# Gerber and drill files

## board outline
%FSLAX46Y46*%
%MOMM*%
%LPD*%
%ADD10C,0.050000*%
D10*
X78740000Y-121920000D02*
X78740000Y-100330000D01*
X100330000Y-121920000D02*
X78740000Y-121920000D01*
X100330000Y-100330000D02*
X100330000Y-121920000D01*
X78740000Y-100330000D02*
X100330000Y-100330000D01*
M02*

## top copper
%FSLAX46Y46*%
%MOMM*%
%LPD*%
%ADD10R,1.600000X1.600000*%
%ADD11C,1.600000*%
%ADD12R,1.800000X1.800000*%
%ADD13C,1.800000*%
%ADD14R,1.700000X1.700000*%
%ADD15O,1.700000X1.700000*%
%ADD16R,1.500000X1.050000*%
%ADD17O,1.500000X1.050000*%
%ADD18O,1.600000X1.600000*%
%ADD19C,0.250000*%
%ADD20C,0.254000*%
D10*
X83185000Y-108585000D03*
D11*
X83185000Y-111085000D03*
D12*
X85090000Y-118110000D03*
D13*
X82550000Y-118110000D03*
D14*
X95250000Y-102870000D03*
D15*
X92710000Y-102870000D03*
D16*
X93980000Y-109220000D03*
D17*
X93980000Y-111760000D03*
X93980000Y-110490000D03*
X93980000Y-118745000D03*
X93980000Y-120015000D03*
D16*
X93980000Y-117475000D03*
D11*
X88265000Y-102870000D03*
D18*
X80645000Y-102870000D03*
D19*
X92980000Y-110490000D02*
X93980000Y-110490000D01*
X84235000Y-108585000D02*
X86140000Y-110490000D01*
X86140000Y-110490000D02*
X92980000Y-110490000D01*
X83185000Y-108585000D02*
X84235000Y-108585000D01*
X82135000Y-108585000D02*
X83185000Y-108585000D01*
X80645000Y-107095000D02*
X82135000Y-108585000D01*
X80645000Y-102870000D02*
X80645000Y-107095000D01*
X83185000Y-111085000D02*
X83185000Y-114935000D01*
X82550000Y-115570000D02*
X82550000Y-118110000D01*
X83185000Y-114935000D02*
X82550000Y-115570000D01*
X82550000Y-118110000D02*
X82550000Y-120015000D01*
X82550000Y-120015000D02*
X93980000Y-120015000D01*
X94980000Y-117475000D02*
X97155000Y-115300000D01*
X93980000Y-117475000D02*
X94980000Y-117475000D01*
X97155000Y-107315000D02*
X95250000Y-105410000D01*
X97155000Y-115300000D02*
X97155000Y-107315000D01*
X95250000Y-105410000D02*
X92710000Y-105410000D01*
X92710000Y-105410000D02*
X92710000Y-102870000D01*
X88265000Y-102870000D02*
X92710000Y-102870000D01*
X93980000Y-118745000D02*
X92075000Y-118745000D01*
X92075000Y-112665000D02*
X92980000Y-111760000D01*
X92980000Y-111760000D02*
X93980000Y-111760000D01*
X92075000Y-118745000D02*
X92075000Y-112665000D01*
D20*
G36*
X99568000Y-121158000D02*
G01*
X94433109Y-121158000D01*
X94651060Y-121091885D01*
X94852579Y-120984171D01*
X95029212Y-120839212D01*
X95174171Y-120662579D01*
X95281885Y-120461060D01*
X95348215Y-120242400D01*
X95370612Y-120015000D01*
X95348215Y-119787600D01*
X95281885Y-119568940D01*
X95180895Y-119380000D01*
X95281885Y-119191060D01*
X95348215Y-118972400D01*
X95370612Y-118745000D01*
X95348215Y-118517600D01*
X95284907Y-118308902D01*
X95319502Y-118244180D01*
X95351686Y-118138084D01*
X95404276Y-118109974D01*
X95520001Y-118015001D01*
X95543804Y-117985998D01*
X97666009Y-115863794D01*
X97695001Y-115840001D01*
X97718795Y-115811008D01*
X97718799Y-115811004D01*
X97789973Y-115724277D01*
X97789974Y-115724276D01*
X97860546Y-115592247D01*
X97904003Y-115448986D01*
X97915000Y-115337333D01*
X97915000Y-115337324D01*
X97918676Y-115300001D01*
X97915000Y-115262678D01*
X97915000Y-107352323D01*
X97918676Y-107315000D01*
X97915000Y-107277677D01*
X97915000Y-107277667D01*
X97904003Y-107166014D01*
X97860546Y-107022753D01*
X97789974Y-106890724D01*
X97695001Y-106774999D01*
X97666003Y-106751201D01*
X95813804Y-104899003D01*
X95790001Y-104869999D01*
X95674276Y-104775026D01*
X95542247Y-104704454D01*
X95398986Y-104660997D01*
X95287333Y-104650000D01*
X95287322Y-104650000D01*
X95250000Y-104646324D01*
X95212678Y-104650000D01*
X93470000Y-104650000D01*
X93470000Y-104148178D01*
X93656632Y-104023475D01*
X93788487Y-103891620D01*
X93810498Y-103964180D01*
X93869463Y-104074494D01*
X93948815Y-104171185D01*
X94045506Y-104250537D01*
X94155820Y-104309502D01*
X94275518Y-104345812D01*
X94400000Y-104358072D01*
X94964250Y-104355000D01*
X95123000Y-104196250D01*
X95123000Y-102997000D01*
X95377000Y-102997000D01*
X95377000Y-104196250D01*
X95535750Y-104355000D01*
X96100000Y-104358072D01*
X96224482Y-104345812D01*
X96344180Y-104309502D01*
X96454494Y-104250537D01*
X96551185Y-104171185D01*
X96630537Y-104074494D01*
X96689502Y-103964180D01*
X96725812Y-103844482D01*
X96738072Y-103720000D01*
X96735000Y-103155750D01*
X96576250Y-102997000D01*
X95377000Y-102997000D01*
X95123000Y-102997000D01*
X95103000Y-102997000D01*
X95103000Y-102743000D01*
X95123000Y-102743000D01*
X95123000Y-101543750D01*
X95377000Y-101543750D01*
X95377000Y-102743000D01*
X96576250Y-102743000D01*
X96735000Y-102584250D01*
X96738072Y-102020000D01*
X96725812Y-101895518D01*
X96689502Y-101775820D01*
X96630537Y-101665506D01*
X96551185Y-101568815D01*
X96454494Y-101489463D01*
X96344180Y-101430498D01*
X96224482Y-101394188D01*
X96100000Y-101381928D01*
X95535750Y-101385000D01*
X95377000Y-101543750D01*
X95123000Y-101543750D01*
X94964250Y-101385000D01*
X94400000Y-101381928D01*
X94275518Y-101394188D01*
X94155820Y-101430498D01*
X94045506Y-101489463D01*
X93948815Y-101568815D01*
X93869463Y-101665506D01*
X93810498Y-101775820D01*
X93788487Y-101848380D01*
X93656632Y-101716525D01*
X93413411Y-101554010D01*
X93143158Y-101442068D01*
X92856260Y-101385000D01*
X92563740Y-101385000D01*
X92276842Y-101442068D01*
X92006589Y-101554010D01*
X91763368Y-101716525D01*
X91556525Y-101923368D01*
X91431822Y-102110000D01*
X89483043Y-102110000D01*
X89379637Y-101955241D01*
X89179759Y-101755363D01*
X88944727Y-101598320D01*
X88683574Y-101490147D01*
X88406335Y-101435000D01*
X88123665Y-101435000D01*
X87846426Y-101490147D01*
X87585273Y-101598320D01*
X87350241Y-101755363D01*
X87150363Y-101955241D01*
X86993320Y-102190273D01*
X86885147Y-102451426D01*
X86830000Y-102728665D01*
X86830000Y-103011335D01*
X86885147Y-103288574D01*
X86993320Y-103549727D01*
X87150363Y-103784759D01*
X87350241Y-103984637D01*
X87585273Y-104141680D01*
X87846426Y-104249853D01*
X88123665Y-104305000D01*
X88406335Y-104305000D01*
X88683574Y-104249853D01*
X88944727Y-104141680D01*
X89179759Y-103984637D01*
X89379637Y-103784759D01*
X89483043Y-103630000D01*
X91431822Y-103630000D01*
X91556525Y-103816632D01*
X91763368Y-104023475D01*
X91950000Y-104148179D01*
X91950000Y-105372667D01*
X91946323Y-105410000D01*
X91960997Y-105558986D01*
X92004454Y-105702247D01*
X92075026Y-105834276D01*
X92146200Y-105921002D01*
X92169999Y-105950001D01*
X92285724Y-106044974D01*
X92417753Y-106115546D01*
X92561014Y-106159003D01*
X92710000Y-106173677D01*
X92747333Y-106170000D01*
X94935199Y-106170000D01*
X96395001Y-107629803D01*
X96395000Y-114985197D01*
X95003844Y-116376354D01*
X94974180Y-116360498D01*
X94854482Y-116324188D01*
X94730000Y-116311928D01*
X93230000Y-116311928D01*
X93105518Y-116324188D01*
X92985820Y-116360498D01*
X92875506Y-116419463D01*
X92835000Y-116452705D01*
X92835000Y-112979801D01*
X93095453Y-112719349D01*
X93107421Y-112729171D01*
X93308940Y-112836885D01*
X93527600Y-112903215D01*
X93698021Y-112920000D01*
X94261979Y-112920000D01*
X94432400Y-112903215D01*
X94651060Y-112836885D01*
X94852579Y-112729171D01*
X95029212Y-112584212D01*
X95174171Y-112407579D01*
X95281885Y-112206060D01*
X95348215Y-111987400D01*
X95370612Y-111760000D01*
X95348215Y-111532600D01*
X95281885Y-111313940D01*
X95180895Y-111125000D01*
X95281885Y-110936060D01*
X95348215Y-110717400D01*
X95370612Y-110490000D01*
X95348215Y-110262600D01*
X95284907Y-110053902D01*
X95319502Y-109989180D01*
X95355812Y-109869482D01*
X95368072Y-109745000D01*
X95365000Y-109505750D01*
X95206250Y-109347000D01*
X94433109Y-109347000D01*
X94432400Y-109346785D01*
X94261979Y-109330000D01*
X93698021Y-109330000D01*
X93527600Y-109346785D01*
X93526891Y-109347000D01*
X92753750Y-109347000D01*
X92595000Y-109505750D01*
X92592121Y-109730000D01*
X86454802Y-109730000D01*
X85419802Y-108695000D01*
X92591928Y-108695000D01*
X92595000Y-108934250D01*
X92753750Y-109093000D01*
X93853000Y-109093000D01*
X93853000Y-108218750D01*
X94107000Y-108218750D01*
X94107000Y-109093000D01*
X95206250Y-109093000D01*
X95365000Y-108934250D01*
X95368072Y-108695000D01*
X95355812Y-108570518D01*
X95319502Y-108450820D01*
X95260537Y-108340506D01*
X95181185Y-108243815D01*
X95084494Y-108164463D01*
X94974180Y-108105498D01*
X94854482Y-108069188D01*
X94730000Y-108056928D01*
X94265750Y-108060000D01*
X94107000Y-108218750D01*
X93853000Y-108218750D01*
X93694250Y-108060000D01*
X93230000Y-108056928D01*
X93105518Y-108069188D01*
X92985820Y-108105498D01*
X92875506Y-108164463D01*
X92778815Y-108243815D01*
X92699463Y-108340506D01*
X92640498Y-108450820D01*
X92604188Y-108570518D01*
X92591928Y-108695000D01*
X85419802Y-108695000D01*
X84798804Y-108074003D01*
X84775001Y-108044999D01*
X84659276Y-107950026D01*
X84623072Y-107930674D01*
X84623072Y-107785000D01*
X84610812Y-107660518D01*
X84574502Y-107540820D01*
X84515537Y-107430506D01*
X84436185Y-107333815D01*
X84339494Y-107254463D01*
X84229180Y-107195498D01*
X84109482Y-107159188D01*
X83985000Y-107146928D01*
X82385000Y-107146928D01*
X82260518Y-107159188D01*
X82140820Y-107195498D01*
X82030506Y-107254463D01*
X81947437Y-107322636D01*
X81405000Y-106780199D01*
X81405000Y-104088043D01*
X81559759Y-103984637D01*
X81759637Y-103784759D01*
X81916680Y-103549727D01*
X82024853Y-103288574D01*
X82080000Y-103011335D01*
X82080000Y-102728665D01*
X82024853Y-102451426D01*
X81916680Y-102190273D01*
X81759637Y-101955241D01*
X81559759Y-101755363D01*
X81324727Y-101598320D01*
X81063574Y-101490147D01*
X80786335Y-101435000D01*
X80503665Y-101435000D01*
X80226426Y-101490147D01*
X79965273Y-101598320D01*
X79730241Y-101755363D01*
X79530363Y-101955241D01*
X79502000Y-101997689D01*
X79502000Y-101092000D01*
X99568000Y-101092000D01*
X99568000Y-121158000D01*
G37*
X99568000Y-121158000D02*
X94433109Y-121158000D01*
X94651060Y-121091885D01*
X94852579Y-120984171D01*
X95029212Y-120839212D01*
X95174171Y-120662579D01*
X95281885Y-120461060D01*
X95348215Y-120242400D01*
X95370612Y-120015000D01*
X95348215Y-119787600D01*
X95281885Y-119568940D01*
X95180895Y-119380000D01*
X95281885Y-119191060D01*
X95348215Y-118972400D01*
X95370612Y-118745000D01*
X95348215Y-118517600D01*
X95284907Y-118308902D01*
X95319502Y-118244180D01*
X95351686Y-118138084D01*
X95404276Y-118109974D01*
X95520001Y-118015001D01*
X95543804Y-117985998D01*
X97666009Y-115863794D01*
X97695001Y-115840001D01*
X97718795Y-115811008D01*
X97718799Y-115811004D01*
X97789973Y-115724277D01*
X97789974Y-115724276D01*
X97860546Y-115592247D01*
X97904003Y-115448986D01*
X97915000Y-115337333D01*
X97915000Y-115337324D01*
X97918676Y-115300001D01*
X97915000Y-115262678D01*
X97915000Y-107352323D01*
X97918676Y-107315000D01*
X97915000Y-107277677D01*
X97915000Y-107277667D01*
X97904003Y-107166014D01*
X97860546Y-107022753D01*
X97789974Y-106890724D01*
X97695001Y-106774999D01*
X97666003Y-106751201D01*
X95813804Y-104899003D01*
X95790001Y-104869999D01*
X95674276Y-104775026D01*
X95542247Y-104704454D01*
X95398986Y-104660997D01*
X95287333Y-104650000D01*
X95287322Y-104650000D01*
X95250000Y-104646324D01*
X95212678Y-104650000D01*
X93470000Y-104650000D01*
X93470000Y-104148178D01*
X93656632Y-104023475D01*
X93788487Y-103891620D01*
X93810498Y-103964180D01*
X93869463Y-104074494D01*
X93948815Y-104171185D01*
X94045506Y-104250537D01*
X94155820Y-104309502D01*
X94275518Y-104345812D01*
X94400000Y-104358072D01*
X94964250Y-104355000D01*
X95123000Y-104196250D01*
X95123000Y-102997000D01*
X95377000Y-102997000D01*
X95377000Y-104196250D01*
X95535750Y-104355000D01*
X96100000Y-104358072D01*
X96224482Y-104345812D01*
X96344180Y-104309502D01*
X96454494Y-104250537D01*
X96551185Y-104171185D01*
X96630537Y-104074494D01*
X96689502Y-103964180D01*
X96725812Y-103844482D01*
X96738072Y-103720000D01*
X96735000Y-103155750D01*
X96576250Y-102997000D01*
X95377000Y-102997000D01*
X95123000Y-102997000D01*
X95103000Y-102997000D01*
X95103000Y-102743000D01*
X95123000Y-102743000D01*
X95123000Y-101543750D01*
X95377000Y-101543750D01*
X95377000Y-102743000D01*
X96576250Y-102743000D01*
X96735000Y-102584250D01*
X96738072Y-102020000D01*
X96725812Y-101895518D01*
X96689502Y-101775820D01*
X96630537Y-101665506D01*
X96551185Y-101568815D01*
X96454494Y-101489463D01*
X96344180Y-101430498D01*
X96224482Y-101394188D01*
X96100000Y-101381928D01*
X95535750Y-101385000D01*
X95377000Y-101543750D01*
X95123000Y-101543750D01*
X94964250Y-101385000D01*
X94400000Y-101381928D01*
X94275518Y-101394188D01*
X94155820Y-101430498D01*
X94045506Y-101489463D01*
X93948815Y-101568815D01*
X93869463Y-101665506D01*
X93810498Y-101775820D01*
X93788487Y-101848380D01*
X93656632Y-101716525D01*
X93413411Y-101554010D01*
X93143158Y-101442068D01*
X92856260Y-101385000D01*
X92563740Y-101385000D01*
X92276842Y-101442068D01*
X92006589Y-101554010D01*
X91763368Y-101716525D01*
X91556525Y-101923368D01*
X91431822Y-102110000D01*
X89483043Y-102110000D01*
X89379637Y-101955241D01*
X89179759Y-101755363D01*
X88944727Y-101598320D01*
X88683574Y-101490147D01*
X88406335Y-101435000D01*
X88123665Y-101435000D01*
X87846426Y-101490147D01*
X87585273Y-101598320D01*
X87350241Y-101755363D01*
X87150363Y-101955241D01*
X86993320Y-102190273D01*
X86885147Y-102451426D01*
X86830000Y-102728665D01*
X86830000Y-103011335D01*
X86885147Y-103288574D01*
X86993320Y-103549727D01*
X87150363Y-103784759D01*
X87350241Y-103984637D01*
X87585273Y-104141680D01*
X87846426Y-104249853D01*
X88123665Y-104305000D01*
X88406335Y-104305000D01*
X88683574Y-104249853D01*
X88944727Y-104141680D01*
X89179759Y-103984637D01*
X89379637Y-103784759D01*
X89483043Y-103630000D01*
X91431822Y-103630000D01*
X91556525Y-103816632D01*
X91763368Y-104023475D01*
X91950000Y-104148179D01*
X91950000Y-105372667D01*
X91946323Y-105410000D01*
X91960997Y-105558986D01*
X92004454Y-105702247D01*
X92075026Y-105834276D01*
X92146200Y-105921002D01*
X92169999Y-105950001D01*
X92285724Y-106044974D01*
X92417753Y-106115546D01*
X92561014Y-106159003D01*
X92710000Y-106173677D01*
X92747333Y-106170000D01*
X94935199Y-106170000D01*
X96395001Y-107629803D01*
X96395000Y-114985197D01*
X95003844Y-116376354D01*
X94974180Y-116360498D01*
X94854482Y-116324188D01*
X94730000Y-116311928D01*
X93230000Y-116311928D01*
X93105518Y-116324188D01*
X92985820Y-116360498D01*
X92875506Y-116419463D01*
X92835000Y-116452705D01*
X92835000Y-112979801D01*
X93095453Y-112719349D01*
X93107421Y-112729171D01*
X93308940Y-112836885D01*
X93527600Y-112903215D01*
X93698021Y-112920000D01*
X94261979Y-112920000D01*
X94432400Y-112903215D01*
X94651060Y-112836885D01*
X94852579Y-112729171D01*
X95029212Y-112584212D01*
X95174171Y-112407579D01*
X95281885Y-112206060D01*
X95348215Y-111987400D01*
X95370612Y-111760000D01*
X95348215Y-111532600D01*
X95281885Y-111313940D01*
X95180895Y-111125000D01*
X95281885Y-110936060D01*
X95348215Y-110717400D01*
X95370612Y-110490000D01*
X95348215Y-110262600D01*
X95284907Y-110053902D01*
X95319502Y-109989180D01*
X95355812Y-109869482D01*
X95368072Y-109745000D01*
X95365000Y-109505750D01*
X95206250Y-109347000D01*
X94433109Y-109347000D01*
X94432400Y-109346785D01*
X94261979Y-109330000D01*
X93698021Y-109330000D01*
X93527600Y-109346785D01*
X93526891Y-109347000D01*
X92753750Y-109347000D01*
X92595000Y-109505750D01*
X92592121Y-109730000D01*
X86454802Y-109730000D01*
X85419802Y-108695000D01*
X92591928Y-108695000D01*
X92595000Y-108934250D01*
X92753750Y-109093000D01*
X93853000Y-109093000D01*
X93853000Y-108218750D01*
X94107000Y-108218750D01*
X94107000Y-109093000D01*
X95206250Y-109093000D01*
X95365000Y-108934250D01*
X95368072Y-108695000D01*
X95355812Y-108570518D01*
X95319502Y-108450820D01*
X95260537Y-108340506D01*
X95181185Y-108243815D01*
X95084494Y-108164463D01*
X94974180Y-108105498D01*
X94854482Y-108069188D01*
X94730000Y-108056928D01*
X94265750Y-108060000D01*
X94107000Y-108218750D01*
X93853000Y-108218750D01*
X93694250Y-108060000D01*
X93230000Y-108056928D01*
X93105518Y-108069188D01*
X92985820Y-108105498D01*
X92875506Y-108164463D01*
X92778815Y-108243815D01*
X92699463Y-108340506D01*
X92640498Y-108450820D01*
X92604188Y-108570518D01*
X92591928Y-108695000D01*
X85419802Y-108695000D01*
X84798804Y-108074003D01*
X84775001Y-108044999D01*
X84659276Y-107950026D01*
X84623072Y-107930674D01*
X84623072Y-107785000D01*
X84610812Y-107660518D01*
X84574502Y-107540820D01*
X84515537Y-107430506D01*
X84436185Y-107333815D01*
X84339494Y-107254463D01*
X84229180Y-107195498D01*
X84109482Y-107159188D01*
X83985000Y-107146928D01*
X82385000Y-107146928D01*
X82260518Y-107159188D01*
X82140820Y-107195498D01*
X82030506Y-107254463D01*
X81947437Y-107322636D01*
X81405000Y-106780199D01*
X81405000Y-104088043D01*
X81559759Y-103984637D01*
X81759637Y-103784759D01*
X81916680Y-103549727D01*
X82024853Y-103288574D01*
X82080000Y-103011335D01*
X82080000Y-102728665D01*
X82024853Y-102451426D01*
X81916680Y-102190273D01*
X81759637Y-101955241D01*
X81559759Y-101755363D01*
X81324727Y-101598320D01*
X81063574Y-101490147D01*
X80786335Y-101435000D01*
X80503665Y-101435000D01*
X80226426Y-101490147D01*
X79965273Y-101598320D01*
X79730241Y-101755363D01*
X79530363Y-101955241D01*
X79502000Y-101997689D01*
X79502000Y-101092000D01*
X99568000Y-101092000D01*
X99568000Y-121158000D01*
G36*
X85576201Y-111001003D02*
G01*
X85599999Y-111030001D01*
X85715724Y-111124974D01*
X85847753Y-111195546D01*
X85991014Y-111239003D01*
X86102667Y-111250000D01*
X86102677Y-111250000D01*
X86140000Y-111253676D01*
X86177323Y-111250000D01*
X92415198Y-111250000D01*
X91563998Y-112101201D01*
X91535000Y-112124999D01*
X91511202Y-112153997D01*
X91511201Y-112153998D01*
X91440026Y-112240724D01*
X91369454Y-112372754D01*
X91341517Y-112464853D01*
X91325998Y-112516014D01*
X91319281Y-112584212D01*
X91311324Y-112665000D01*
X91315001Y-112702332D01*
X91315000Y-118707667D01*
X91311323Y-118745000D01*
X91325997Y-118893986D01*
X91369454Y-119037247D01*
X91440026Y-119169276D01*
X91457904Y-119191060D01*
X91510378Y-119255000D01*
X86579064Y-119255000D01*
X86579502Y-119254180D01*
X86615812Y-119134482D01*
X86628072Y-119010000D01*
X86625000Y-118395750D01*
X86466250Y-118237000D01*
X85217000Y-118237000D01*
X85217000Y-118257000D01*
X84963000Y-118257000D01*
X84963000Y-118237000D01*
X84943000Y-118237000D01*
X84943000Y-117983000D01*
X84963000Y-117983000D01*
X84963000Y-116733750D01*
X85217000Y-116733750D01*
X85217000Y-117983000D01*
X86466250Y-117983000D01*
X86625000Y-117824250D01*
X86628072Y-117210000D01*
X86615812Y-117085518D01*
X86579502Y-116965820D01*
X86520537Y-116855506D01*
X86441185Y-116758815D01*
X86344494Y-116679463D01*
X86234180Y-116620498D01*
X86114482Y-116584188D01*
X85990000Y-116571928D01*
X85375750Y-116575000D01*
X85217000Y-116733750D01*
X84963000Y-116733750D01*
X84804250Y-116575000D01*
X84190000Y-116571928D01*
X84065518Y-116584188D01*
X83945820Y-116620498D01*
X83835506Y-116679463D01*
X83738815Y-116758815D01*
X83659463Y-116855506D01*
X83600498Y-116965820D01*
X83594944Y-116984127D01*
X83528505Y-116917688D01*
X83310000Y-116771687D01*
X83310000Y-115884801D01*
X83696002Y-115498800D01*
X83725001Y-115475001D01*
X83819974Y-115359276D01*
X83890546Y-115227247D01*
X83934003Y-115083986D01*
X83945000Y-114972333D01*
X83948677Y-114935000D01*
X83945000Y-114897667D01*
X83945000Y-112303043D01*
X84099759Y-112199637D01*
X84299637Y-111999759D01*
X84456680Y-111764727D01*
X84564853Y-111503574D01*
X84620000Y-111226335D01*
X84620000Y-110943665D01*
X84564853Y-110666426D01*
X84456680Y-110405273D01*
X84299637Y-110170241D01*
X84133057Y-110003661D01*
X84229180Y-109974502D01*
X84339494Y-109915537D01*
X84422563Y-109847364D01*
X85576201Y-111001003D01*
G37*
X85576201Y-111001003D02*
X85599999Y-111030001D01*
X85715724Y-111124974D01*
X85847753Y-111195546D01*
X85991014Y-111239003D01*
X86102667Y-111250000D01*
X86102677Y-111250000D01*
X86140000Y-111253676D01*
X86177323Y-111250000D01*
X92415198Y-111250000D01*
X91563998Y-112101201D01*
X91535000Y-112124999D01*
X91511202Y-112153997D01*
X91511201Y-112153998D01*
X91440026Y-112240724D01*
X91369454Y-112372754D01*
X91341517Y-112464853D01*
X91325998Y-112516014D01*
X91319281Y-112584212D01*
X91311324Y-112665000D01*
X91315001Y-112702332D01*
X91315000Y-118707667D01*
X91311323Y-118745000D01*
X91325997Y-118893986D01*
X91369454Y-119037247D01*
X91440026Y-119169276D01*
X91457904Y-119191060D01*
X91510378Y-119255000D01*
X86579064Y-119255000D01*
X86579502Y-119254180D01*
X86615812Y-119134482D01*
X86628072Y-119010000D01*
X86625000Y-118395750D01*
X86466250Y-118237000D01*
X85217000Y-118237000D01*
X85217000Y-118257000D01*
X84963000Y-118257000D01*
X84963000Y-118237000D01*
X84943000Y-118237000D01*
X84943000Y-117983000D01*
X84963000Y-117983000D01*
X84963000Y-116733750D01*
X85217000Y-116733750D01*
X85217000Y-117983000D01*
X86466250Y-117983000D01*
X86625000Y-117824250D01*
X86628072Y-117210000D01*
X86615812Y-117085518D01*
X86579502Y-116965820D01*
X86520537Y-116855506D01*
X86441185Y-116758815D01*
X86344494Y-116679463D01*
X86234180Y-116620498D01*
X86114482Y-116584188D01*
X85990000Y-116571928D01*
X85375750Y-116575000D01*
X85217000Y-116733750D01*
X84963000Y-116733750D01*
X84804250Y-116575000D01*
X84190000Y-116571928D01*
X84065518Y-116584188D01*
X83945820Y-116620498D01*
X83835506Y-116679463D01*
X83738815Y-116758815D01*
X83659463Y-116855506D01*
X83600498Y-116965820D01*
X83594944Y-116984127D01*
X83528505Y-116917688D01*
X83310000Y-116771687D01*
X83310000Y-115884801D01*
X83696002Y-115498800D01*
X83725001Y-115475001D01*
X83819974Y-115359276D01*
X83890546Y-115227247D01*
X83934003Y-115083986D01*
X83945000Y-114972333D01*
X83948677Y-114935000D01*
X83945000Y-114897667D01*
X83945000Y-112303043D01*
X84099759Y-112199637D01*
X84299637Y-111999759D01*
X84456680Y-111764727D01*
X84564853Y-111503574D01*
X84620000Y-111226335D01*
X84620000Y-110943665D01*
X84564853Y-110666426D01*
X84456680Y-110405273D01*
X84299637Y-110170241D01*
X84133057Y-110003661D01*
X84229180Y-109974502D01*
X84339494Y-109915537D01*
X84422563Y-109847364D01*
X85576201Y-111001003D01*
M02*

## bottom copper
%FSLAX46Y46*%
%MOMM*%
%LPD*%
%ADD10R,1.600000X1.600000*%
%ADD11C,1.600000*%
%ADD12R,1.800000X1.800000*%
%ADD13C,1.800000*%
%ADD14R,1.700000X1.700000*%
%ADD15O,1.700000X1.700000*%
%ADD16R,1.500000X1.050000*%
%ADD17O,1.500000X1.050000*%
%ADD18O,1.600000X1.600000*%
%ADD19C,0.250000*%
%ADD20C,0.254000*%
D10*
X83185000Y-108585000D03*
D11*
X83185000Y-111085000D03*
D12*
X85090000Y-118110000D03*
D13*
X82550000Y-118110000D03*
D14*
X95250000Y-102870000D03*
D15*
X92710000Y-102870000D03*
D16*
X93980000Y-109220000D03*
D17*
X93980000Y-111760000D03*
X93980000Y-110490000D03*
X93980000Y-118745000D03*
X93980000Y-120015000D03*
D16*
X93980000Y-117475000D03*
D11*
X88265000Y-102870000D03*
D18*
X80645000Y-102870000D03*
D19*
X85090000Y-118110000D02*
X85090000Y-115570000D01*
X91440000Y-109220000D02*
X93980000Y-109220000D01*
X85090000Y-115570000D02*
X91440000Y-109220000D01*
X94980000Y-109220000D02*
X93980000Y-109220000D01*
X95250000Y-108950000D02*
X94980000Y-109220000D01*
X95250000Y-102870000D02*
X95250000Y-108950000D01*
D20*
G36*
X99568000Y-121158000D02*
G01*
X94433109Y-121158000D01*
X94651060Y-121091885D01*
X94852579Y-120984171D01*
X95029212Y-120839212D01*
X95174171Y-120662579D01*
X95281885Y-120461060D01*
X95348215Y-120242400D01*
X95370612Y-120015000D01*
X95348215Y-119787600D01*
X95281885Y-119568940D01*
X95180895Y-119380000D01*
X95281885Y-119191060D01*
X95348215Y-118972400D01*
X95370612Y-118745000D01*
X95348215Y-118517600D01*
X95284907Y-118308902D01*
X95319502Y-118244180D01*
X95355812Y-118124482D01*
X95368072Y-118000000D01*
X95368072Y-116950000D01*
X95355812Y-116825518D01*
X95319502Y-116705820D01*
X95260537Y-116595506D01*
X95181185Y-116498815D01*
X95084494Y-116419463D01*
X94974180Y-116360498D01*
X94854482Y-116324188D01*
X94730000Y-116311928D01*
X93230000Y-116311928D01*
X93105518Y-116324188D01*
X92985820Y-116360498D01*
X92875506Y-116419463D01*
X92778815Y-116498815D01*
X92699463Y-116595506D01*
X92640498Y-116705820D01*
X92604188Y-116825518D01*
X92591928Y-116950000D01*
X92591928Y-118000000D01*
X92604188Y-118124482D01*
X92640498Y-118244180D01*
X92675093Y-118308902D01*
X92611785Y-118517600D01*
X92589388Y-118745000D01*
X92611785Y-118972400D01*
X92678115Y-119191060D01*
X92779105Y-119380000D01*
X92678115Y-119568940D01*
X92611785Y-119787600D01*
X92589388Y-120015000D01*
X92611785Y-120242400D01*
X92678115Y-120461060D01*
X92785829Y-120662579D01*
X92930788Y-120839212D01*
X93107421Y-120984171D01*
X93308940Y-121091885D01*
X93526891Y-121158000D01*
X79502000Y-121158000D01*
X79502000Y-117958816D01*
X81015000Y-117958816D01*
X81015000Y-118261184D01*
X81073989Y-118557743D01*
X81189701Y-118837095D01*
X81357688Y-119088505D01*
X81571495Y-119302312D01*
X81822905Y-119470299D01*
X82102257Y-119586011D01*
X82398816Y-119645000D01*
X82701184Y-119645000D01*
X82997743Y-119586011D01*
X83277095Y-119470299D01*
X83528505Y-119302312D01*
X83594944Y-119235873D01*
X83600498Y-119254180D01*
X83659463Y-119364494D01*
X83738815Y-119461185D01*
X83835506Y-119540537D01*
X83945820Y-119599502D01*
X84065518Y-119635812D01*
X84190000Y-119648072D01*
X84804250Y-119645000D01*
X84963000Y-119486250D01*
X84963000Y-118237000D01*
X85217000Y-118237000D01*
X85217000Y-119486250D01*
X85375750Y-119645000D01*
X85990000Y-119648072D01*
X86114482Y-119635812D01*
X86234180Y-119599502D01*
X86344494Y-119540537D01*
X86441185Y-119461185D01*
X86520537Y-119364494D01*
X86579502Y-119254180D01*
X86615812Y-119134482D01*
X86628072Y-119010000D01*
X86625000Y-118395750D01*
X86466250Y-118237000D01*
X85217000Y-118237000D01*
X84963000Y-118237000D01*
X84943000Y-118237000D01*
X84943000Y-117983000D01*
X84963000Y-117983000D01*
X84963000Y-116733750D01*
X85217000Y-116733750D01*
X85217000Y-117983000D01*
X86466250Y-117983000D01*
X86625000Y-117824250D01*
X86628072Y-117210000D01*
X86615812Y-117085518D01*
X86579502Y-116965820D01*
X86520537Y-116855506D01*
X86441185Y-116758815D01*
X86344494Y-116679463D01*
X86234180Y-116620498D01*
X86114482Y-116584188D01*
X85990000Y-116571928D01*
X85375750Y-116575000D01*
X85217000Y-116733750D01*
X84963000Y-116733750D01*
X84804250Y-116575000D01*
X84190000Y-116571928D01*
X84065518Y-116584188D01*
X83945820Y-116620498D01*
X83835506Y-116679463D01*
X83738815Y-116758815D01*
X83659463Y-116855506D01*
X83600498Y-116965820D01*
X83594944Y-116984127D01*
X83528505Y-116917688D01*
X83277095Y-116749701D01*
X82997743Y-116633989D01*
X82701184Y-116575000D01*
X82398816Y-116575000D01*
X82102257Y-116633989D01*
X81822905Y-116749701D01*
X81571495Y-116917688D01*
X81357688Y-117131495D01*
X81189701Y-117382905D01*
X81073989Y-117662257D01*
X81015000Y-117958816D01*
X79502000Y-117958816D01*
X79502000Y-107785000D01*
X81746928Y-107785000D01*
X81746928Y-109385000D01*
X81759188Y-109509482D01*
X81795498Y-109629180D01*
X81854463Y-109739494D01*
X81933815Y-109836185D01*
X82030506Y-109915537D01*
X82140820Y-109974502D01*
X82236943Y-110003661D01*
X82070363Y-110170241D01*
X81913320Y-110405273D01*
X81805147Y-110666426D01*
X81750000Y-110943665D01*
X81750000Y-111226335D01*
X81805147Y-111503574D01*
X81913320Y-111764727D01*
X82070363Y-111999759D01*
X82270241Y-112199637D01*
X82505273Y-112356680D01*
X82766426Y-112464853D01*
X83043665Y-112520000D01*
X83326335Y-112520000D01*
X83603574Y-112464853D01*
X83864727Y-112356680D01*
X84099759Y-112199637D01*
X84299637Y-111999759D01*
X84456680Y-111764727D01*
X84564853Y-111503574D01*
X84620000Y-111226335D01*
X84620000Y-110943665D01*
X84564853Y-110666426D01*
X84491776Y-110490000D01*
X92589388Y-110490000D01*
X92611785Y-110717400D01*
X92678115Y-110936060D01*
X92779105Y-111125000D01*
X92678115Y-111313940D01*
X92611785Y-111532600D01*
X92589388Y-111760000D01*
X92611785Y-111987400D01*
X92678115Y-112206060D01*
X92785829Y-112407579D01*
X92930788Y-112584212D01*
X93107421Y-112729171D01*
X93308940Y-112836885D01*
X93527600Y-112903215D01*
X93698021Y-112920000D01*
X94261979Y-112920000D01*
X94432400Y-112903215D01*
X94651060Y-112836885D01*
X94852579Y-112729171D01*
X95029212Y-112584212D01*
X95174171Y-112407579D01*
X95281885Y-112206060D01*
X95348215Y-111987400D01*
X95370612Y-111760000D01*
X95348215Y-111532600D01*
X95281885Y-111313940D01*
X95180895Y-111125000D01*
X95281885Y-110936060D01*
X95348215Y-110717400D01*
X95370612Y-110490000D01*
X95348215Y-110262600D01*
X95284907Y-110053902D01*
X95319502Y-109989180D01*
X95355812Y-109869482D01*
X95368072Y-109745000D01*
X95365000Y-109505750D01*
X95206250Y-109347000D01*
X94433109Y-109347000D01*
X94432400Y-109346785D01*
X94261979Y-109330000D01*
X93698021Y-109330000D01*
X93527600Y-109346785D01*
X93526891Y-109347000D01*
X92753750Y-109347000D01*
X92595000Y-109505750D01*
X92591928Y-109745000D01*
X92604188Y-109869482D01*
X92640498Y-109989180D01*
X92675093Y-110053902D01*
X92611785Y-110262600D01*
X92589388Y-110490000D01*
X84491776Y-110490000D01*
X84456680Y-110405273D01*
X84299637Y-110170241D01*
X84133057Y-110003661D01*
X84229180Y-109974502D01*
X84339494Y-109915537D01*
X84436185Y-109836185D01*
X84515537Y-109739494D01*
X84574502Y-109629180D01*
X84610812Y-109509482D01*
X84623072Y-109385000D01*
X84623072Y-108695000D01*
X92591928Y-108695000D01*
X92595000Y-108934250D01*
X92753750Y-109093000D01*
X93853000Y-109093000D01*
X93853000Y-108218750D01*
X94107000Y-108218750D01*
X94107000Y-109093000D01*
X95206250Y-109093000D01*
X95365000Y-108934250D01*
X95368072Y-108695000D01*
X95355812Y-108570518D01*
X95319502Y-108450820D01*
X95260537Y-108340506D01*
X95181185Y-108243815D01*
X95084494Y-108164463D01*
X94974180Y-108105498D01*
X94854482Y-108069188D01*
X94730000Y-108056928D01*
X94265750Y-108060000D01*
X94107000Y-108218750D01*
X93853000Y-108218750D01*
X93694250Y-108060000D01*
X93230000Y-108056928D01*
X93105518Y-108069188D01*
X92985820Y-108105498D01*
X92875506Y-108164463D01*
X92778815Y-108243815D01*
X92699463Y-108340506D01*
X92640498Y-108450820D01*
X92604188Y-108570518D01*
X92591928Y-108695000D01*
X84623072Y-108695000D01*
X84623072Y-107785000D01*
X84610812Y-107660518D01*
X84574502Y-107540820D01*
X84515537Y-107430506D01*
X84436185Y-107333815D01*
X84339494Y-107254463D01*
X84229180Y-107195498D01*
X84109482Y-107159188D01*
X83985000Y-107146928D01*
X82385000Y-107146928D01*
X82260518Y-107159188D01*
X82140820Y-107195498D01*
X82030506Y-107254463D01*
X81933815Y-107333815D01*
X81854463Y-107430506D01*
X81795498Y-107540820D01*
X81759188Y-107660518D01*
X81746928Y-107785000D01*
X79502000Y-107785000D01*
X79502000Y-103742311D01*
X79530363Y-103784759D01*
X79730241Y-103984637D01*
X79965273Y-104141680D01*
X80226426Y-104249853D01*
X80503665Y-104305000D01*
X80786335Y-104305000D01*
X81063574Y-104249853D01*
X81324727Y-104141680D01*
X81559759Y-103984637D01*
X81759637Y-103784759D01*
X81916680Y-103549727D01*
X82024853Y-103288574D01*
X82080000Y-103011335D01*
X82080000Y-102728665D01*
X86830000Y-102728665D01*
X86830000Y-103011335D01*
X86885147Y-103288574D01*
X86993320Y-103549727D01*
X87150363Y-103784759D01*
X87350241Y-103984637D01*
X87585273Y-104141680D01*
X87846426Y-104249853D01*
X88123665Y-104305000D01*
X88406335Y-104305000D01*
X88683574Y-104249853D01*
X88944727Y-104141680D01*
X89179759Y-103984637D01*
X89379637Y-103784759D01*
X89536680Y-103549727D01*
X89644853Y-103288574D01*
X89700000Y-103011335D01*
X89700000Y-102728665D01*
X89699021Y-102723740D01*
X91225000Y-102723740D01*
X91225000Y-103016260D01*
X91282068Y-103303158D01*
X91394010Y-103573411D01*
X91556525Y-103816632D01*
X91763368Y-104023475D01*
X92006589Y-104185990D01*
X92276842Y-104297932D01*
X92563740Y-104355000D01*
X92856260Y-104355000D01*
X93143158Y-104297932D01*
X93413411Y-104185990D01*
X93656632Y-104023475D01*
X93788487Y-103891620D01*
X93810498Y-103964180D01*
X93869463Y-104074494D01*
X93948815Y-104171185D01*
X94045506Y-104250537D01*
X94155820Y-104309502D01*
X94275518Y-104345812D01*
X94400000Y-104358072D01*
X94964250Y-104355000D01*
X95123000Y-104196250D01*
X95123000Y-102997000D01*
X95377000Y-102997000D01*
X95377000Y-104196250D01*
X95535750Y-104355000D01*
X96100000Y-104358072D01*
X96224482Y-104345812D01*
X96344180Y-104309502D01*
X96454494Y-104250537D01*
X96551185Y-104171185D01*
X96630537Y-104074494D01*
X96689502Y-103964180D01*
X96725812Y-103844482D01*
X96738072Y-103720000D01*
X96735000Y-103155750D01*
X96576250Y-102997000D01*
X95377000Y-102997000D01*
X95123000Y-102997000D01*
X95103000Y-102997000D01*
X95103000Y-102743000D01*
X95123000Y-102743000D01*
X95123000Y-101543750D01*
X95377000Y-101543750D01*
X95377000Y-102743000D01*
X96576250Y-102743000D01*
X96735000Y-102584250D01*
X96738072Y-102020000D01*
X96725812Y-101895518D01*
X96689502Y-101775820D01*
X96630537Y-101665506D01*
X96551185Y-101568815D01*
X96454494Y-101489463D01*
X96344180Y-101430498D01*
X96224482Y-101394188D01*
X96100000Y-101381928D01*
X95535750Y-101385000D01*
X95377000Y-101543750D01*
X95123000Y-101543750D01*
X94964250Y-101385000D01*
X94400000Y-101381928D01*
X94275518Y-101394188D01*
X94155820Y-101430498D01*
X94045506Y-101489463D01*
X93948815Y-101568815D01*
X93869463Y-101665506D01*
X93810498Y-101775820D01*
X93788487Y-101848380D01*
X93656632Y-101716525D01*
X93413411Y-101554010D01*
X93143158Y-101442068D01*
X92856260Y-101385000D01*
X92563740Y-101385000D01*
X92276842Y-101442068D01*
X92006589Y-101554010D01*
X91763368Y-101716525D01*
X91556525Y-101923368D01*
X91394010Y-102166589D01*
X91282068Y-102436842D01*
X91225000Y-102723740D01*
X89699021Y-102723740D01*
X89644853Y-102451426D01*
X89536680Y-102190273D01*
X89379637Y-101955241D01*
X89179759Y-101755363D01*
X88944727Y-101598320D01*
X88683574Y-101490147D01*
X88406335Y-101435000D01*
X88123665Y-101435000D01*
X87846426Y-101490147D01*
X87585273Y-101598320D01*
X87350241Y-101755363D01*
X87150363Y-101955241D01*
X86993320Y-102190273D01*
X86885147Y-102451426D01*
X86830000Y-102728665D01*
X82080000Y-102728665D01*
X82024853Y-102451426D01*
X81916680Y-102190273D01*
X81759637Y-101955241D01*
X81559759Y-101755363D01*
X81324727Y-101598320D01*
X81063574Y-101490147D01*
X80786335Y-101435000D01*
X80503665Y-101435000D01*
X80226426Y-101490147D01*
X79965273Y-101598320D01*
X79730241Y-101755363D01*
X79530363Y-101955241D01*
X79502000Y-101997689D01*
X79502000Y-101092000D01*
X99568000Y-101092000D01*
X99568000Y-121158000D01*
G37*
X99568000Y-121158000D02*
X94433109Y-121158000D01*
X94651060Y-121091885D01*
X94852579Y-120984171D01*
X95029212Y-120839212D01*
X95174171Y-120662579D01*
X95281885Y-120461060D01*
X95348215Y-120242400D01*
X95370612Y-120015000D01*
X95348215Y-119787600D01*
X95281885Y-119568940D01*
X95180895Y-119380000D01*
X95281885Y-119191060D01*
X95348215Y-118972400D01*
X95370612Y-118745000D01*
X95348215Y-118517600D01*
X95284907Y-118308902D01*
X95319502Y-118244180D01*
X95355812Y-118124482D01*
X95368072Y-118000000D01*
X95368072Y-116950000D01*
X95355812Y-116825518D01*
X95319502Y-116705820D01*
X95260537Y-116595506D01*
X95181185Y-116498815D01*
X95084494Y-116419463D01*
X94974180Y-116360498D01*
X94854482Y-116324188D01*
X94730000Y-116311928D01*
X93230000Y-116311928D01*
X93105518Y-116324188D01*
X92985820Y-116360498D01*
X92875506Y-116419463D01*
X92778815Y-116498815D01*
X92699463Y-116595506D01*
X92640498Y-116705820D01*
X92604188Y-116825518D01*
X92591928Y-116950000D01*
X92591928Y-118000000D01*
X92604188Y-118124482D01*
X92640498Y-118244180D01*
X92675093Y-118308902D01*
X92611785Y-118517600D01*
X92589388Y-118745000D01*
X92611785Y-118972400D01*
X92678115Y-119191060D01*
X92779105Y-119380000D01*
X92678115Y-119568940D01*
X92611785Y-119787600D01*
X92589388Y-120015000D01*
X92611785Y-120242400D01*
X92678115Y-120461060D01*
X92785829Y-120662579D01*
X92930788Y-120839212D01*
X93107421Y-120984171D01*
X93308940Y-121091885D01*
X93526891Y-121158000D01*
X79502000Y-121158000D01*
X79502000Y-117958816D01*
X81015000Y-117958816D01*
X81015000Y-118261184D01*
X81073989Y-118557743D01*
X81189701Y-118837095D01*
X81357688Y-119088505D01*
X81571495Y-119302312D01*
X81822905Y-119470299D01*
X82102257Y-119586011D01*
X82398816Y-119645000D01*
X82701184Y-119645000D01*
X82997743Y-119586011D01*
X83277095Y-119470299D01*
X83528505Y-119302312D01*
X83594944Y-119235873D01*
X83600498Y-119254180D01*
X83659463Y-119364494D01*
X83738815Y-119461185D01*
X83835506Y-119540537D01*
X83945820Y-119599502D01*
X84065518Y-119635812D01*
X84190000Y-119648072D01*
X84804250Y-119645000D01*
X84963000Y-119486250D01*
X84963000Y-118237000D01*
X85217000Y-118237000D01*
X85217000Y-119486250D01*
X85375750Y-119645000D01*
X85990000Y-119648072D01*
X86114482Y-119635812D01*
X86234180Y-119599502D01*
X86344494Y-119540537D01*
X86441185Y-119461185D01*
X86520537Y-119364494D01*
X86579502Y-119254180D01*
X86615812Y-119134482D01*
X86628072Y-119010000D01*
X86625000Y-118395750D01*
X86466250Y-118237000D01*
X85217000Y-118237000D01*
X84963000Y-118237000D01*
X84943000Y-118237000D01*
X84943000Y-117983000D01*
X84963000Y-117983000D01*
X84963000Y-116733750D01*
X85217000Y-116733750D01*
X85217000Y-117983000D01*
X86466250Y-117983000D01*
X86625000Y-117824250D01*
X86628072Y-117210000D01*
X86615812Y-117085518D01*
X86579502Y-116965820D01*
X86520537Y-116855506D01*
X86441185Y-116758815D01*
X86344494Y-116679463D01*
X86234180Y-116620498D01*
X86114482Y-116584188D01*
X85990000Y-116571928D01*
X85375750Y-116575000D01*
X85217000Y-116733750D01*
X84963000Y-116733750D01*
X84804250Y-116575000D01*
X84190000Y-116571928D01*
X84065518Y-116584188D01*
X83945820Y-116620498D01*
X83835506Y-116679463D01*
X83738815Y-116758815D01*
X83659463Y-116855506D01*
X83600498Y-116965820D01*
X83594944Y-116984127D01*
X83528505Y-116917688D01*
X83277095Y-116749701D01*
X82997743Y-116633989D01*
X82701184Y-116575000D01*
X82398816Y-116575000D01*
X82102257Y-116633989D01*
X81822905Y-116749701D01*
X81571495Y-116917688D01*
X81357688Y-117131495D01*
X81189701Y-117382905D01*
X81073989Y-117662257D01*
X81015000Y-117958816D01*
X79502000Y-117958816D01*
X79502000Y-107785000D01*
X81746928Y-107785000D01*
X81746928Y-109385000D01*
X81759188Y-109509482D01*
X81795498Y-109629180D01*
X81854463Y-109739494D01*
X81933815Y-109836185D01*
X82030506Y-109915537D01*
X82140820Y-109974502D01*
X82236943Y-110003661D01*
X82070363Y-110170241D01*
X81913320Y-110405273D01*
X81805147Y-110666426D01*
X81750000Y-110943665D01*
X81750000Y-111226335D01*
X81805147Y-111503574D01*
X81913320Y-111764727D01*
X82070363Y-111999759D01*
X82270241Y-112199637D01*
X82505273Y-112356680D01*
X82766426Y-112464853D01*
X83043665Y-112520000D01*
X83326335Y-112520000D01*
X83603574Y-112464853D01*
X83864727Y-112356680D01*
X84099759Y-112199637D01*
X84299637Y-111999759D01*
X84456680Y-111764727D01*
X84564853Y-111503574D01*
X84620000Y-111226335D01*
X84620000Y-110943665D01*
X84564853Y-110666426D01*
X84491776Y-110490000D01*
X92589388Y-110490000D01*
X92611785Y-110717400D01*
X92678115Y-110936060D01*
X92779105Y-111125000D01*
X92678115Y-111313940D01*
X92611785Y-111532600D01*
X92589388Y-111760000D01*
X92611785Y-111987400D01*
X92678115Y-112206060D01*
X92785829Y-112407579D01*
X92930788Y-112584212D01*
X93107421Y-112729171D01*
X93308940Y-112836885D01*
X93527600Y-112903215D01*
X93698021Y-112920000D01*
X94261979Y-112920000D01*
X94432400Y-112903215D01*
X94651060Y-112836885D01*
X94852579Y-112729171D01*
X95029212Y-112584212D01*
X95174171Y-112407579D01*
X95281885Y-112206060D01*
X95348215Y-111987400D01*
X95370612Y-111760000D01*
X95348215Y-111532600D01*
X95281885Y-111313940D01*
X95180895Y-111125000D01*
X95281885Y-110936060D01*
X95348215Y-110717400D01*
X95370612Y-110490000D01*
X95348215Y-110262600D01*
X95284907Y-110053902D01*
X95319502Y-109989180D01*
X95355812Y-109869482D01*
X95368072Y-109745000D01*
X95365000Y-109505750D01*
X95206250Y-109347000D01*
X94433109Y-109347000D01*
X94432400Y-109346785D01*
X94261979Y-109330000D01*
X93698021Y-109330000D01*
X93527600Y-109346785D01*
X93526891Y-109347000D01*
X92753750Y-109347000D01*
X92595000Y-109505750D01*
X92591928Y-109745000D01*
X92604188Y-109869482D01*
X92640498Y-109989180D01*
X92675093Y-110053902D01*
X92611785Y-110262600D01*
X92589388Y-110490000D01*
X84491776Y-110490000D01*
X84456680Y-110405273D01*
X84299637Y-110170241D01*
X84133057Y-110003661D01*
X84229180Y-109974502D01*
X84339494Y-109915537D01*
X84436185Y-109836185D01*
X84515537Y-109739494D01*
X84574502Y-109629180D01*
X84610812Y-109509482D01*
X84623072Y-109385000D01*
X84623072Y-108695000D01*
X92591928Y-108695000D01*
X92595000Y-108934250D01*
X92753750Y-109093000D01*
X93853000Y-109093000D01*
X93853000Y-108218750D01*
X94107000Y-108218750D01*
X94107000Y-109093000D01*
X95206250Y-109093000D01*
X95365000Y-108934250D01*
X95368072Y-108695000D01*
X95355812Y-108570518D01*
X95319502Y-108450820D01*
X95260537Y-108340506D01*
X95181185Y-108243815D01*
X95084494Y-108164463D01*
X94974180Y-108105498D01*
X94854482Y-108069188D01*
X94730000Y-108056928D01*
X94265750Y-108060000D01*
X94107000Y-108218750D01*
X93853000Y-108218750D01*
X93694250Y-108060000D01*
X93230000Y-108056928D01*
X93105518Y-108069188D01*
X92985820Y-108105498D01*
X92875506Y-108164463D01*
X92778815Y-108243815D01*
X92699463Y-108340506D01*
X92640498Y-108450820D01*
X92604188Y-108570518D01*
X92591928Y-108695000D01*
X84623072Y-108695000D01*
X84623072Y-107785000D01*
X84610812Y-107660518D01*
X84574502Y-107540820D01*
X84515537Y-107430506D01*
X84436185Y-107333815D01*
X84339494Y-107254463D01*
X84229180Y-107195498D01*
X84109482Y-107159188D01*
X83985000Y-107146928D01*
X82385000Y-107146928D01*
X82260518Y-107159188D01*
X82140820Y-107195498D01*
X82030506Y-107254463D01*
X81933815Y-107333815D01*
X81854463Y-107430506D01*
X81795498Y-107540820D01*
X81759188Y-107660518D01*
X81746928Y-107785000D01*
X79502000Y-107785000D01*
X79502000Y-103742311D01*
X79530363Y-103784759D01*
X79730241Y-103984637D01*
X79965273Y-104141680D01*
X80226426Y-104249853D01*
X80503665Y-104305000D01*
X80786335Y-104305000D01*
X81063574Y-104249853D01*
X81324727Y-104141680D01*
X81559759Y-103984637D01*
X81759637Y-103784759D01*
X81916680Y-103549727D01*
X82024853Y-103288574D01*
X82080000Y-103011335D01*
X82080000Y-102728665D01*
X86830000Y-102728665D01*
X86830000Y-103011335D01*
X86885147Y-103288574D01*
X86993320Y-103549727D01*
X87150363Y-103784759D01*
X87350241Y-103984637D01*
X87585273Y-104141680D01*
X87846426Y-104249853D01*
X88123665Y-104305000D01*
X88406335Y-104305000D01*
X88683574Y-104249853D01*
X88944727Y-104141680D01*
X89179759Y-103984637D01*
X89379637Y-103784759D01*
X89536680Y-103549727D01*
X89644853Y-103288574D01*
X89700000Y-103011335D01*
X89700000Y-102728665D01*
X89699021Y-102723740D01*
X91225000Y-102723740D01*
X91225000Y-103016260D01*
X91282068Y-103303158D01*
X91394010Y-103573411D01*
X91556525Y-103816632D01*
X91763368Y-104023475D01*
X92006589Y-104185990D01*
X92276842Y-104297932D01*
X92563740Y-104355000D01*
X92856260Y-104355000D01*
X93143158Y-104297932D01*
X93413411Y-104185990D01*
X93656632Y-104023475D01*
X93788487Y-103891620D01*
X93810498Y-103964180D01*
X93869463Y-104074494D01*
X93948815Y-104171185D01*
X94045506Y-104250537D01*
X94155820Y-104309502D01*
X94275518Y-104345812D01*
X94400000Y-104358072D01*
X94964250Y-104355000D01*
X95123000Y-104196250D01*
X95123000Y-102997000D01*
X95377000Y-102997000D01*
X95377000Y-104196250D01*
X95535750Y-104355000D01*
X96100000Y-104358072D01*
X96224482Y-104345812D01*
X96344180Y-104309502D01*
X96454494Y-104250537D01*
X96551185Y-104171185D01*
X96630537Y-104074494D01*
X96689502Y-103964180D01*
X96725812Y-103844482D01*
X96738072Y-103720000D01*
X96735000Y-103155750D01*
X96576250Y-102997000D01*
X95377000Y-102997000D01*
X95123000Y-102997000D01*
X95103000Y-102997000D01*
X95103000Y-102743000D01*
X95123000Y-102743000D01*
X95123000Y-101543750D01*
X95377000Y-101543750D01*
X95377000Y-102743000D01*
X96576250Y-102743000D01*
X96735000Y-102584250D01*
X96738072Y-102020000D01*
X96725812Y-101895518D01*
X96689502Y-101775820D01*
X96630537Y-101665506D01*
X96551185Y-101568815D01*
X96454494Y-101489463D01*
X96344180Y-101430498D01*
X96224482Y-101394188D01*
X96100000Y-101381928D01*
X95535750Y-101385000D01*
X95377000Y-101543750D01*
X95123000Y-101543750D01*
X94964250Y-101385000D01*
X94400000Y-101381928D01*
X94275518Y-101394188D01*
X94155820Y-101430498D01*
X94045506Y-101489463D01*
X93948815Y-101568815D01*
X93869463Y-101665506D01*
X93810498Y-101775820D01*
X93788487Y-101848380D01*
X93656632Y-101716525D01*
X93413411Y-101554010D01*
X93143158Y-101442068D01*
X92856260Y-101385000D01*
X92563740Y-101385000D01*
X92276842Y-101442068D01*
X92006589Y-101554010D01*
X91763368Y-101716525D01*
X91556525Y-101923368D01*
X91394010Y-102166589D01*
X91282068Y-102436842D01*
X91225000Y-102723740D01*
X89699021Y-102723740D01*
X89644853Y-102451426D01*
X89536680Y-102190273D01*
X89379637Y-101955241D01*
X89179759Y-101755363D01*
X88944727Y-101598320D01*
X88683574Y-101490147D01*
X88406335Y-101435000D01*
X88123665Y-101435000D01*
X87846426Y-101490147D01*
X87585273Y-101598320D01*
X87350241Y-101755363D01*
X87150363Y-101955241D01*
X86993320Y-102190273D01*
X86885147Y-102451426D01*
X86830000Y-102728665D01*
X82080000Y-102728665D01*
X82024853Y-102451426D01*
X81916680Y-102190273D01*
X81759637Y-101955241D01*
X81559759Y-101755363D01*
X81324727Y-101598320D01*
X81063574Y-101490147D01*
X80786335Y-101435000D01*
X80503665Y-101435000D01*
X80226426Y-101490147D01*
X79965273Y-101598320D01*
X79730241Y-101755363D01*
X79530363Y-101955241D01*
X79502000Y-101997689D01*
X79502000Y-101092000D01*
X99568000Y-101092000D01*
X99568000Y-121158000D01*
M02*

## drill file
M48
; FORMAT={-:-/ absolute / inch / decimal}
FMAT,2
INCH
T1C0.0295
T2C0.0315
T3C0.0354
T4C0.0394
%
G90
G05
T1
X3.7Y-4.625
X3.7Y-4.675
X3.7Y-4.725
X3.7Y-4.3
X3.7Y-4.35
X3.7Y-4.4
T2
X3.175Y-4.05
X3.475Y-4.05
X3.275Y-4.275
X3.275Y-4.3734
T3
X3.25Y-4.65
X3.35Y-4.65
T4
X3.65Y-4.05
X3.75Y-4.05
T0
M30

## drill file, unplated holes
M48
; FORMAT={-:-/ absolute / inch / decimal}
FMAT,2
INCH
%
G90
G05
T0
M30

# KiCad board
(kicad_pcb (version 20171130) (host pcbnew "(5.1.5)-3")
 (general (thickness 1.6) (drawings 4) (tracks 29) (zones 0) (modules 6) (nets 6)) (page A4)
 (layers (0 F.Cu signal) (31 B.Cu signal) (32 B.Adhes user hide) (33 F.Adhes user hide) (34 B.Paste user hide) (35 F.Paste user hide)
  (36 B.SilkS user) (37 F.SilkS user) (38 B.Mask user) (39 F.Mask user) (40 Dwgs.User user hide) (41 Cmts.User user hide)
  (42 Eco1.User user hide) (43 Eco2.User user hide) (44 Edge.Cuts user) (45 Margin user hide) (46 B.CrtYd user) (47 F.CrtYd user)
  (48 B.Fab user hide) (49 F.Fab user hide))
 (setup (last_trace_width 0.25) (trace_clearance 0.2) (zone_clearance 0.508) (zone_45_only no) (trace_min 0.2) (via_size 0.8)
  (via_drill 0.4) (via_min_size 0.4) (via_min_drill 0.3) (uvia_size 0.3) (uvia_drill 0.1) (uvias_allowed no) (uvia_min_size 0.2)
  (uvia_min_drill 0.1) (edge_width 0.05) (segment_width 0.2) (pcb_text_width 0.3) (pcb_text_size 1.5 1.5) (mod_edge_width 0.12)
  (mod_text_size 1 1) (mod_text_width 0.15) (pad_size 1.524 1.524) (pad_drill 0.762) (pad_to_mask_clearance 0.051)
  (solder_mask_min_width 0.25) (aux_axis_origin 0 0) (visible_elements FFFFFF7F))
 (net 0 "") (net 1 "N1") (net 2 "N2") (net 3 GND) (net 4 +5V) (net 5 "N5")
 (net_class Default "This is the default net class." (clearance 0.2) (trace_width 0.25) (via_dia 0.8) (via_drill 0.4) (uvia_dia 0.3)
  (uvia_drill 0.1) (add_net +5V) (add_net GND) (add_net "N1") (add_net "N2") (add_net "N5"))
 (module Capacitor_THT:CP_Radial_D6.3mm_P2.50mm (layer F.Cu) (at 83.185 108.585 270)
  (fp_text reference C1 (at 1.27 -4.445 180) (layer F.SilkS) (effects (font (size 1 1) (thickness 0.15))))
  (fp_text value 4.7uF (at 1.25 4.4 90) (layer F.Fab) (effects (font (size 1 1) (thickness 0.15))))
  (pad 1 thru_hole rect (at 0 0 270) (size 1.6 1.6) (drill 0.8) (layers *.Cu *.Mask) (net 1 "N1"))
  (pad 2 thru_hole circle (at 2.5 0 270) (size 1.6 1.6) (drill 0.8) (layers *.Cu *.Mask) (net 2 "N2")))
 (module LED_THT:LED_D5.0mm (layer F.Cu) (at 85.09 118.11 180)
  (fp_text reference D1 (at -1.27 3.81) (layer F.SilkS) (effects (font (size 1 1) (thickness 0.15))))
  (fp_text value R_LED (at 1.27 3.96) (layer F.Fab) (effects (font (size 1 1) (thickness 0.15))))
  (pad 1 thru_hole rect (at 0 0 180) (size 1.8 1.8) (drill 0.9) (layers *.Cu *.Mask) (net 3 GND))
  (pad 2 thru_hole circle (at 2.54 0 180) (size 1.8 1.8) (drill 0.9) (layers *.Cu *.Mask) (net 2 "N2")))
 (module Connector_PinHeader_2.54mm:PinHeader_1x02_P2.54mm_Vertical (layer F.Cu) (at 95.25 102.87 270)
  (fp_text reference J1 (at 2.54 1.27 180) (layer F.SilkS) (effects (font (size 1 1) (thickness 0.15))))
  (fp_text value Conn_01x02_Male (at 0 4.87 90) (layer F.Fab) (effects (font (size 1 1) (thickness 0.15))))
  (pad 1 thru_hole rect (at 0 0 270) (size 1.7 1.7) (drill 1) (layers *.Cu *.Mask) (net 3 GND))
  (pad 2 thru_hole oval (at 0 2.54 270) (size 1.7 1.7) (drill 1) (layers *.Cu *.Mask) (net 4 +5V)))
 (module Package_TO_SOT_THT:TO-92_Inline (layer F.Cu) (at 93.98 109.22 270)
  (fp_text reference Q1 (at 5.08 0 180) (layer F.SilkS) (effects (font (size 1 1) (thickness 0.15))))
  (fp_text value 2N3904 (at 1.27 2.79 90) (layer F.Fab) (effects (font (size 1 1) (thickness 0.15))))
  (pad 1 thru_hole rect (at 0 0 270) (size 1.05 1.5) (drill 0.75) (layers *.Cu *.Mask) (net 3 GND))
  (pad 3 thru_hole oval (at 2.54 0 270) (size 1.05 1.5) (drill 0.75) (layers *.Cu *.Mask) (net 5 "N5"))
  (pad 2 thru_hole oval (at 1.27 0 270) (size 1.05 1.5) (drill 0.75) (layers *.Cu *.Mask) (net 1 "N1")))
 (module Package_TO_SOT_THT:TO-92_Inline (layer F.Cu) (at 93.98 117.475 270)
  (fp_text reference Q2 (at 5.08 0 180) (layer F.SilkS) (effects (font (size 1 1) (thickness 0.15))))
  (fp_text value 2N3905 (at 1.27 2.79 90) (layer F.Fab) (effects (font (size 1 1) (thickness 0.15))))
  (pad 2 thru_hole oval (at 1.27 0 270) (size 1.05 1.5) (drill 0.75) (layers *.Cu *.Mask) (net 5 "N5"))
  (pad 3 thru_hole oval (at 2.54 0 270) (size 1.05 1.5) (drill 0.75) (layers *.Cu *.Mask) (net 2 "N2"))
  (pad 1 thru_hole rect (at 0 0 270) (size 1.05 1.5) (drill 0.75) (layers *.Cu *.Mask) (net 4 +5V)))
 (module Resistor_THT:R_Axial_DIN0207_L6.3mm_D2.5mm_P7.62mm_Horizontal (layer F.Cu) (at 88.265 102.87 180)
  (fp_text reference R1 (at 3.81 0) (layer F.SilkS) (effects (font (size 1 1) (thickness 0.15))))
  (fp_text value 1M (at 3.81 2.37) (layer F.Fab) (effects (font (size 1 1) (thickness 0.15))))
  (pad 1 thru_hole circle (at 0 0 180) (size 1.6 1.6) (drill 0.8) (layers *.Cu *.Mask) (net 4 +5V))
  (pad 2 thru_hole oval (at 7.62 0 180) (size 1.6 1.6) (drill 0.8) (layers *.Cu *.Mask) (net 1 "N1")))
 (gr_line (start 78.74 121.92) (end 78.74 100.33) (layer Edge.Cuts) (width 0.05))
 (gr_line (start 100.33 121.92) (end 78.74 121.92) (layer Edge.Cuts) (width 0.05))
 (gr_line (start 100.33 100.33) (end 100.33 121.92) (layer Edge.Cuts) (width 0.05))
 (gr_line (start 78.74 100.33) (end 100.33 100.33) (layer Edge.Cuts) (width 0.05))
 (segment (start 92.98 110.49) (end 93.98 110.49) (width 0.25) (layer F.Cu) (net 1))
 (segment (start 84.235 108.585) (end 86.14 110.49) (width 0.25) (layer F.Cu) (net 1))
 (segment (start 86.14 110.49) (end 92.98 110.49) (width 0.25) (layer F.Cu) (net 1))
 (segment (start 83.185 108.585) (end 84.235 108.585) (width 0.25) (layer F.Cu) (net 1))
 (segment (start 82.135 108.585) (end 83.185 108.585) (width 0.25) (layer F.Cu) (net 1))
 (segment (start 80.645 107.095) (end 82.135 108.585) (width 0.25) (layer F.Cu) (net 1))
 (segment (start 80.645 102.87) (end 80.645 107.095) (width 0.25) (layer F.Cu) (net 1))
 (segment (start 83.185 111.085) (end 83.185 114.935) (width 0.25) (layer F.Cu) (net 2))
 (segment (start 82.55 115.57) (end 82.55 118.11) (width 0.25) (layer F.Cu) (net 2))
 (segment (start 83.185 114.935) (end 82.55 115.57) (width 0.25) (layer F.Cu) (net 2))
 (segment (start 82.55 118.11) (end 82.55 120.015) (width 0.25) (layer F.Cu) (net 2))
 (segment (start 82.55 120.015) (end 93.98 120.015) (width 0.25) (layer F.Cu) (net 2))
 (segment (start 85.09 118.11) (end 85.09 115.57) (width 0.25) (layer B.Cu) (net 3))
 (segment (start 91.44 109.22) (end 93.98 109.22) (width 0.25) (layer B.Cu) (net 3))
 (segment (start 85.09 115.57) (end 91.44 109.22) (width 0.25) (layer B.Cu) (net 3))
 (segment (start 94.98 109.22) (end 93.98 109.22) (width 0.25) (layer B.Cu) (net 3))
 (segment (start 95.25 108.95) (end 94.98 109.22) (width 0.25) (layer B.Cu) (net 3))
 (segment (start 95.25 102.87) (end 95.25 108.95) (width 0.25) (layer B.Cu) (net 3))
 (segment (start 94.98 117.475) (end 97.155 115.3) (width 0.25) (layer F.Cu) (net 4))
 (segment (start 93.98 117.475) (end 94.98 117.475) (width 0.25) (layer F.Cu) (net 4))
 (segment (start 97.155 107.315) (end 95.25 105.41) (width 0.25) (layer F.Cu) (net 4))
 (segment (start 97.155 115.3) (end 97.155 107.315) (width 0.25) (layer F.Cu) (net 4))
 (segment (start 95.25 105.41) (end 92.71 105.41) (width 0.25) (layer F.Cu) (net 4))
 (segment (start 92.71 105.41) (end 92.71 102.87) (width 0.25) (layer F.Cu) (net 4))
 (segment (start 88.265 102.87) (end 92.71 102.87) (width 0.25) (layer F.Cu) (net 4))
 (segment (start 93.98 118.745) (end 92.075 118.745) (width 0.25) (layer F.Cu) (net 5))
 (segment (start 92.075 112.665) (end 92.98 111.76) (width 0.25) (layer F.Cu) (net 5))
 (segment (start 92.98 111.76) (end 93.98 111.76) (width 0.25) (layer F.Cu) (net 5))
 (segment (start 92.075 118.745) (end 92.075 112.665) (width 0.25) (layer F.Cu) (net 5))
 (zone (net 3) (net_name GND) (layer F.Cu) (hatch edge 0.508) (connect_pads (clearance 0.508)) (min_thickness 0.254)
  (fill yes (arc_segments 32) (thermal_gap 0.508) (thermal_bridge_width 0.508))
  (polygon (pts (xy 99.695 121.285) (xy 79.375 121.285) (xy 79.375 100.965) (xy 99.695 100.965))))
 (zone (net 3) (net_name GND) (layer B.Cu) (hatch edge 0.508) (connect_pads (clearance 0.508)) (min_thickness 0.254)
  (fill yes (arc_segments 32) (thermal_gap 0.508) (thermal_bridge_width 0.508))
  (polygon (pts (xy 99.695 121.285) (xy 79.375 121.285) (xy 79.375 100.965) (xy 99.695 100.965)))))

